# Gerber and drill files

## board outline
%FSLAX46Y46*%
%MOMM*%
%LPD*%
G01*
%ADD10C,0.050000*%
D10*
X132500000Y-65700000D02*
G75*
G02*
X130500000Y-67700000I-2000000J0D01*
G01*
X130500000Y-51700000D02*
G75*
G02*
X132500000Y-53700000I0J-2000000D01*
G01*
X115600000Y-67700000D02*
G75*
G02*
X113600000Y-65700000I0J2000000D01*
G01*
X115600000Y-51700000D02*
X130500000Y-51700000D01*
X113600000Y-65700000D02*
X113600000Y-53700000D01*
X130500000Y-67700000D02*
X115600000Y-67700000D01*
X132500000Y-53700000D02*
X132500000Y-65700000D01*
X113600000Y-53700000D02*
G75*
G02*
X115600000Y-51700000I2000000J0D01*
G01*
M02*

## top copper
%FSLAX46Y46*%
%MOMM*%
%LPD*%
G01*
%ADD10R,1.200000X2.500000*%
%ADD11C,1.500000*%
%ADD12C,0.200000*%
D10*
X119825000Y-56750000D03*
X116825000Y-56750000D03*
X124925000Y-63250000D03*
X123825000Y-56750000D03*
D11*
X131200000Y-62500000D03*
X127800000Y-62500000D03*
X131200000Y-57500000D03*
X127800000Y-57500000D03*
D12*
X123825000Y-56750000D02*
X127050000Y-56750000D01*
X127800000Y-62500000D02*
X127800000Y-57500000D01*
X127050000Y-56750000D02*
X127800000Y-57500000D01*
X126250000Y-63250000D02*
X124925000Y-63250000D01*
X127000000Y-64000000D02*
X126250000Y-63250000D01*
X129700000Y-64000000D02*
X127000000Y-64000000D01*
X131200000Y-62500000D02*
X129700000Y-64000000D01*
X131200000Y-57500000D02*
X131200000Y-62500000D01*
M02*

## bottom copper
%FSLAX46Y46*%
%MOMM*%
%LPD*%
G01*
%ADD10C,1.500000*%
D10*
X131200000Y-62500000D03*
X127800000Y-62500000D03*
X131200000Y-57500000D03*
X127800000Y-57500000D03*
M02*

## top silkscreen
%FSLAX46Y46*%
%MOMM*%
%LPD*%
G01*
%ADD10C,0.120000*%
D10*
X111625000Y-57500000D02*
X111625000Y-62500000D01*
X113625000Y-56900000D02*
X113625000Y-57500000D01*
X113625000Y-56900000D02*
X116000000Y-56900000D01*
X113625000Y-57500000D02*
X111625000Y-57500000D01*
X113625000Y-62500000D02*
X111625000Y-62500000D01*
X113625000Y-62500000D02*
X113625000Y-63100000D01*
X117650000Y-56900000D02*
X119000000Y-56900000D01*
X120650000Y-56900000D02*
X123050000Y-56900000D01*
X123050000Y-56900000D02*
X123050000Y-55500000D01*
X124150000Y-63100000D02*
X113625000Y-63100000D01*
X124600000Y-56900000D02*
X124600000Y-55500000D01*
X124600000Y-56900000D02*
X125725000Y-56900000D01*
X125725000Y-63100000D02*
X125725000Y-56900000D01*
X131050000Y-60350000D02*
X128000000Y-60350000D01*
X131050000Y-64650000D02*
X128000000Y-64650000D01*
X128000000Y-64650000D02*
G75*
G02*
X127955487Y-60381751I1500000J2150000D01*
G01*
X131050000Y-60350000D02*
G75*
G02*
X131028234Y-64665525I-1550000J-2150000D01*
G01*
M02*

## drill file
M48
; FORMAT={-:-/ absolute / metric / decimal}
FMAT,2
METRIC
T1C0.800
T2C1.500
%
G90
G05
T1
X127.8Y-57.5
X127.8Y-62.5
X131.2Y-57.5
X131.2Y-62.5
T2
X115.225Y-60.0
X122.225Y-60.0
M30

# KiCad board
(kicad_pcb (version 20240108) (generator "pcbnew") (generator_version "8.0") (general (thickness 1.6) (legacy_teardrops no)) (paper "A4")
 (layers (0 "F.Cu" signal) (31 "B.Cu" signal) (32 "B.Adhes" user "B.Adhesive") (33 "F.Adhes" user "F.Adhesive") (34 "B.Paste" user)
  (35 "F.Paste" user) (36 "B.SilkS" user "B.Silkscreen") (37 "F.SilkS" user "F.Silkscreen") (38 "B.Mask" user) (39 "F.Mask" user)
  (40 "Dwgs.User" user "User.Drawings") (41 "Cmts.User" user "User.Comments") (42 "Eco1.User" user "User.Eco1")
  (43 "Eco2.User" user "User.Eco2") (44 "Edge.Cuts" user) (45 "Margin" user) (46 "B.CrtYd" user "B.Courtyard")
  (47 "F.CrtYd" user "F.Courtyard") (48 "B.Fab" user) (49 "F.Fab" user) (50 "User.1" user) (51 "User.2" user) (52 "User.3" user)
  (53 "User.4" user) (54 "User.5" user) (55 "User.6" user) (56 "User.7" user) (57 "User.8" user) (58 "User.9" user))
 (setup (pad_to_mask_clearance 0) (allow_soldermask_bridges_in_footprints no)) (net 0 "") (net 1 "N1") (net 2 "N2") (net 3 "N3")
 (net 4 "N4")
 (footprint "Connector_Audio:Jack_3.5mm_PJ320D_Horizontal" (layer "F.Cu") (at 120 60)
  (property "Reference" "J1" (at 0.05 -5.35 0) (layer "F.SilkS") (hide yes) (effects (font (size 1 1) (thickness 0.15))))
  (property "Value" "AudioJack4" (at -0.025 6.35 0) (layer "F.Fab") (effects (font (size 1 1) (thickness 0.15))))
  (fp_line (start -8.375 -2.5) (end -8.375 2.5) (stroke (width 0.12) (type solid)) (layer "F.SilkS"))
  (fp_line (start -6.375 -3.1) (end -6.375 -2.5) (stroke (width 0.12) (type solid)) (layer "F.SilkS"))
  (fp_line (start -6.375 -3.1) (end -4 -3.1) (stroke (width 0.12) (type solid)) (layer "F.SilkS"))
  (fp_line (start -6.375 -2.5) (end -8.375 -2.5) (stroke (width 0.12) (type solid)) (layer "F.SilkS"))
  (fp_line (start -6.375 2.5) (end -8.375 2.5) (stroke (width 0.12) (type solid)) (layer "F.SilkS"))
  (fp_line (start -6.375 2.5) (end -6.375 3.1) (stroke (width 0.12) (type solid)) (layer "F.SilkS"))
  (fp_line (start -2.35 -3.1) (end -1 -3.1) (stroke (width 0.12) (type solid)) (layer "F.SilkS"))
  (fp_line (start 0.65 -3.1) (end 3.05 -3.1) (stroke (width 0.12) (type solid)) (layer "F.SilkS"))
  (fp_line (start 3.05 -3.1) (end 3.05 -4.5) (stroke (width 0.12) (type solid)) (layer "F.SilkS"))
  (fp_line (start 4.15 3.1) (end -6.375 3.1) (stroke (width 0.12) (type solid)) (layer "F.SilkS"))
  (fp_line (start 4.6 -3.1) (end 4.6 -4.5) (stroke (width 0.12) (type solid)) (layer "F.SilkS"))
  (fp_line (start 4.6 -3.1) (end 5.725 -3.1) (stroke (width 0.12) (type solid)) (layer "F.SilkS"))
  (fp_line (start 5.725 3.1) (end 5.725 -3.1) (stroke (width 0.12) (type solid)) (layer "F.SilkS"))
  (pad "" np_thru_hole circle (at -4.775 0) (size 1.5 1.5) (drill 1.5) (layers "*.Cu" "*.Mask"))
  (pad "" np_thru_hole circle (at 2.225 0) (size 1.5 1.5) (drill 1.5) (layers "*.Cu" "*.Mask"))
  (pad "R1" smd rect (at -0.175 -3.25) (size 1.2 2.5) (layers "F.Cu" "F.Paste" "F.Mask") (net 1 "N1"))
  (pad "R2" smd rect (at -3.175 -3.25) (size 1.2 2.5) (layers "F.Cu" "F.Paste" "F.Mask") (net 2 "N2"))
  (pad "S" smd rect (at 4.925 3.25) (size 1.2 2.5) (layers "F.Cu" "F.Paste" "F.Mask") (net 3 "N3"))
  (pad "T" smd rect (at 3.825 -3.25) (size 1.2 2.5) (layers "F.Cu" "F.Paste" "F.Mask") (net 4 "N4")))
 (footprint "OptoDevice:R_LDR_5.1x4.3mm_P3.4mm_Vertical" (layer "F.Cu") (at 131.2 62.5 180)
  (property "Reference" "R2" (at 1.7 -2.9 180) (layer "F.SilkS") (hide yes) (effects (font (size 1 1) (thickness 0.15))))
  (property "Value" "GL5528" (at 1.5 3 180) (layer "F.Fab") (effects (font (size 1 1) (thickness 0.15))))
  (fp_line (start 0.15 2.15) (end 3.2 2.15) (stroke (width 0.12) (type solid)) (layer "F.SilkS"))
  (fp_line (start 0.15 -2.15) (end 3.2 -2.15) (stroke (width 0.12) (type solid)) (layer "F.SilkS"))
  (fp_arc (start 3.2 -2.15) (mid 4.321403 -0.027338) (end 3.244513 2.118249) (stroke (width 0.12) (type solid)) (layer "F.SilkS"))
  (fp_arc (start 0.15 2.15) (mid -0.950438 -0.013368) (end 0.171766 -2.165525) (stroke (width 0.12) (type solid)) (layer "F.SilkS"))
  (pad "1" thru_hole circle (at 0 0 180) (size 1.5 1.5) (drill 0.8) (layers "*.Cu" "*.Mask") (remove_unused_layers no) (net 3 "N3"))
  (pad "2" thru_hole circle (at 3.4 0 180) (size 1.5 1.5) (drill 0.8) (layers "*.Cu" "*.Mask") (remove_unused_layers no) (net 4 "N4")))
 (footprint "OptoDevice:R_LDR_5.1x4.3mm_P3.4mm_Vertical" (layer "B.Cu") (at 131.2 57.5 180)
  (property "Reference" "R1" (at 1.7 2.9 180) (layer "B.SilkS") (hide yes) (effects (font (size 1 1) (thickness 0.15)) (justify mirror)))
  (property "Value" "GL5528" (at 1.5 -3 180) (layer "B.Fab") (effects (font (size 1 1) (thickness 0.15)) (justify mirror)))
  (pad "1" thru_hole circle (at 0 0 180) (size 1.5 1.5) (drill 0.8) (layers "*.Cu" "*.Mask") (remove_unused_layers no) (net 3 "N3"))
  (pad "2" thru_hole circle (at 3.4 0 180) (size 1.5 1.5) (drill 0.8) (layers "*.Cu" "*.Mask") (remove_unused_layers no) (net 4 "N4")))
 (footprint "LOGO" (layer "B.Cu") (at 120.6 55.7 180)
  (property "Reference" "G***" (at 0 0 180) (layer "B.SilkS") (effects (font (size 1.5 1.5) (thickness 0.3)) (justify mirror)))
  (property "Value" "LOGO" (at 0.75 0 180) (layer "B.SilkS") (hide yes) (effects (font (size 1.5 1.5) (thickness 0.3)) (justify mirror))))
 (gr_arc (start 132.5 65.7) (mid 131.914214 67.114214) (end 130.5 67.7) (stroke (width 0.05) (type default)) (layer "Edge.Cuts"))
 (gr_arc (start 130.5 51.7) (mid 131.914214 52.285786) (end 132.5 53.7) (stroke (width 0.05) (type default)) (layer "Edge.Cuts"))
 (gr_arc (start 115.6 67.7) (mid 114.185786 67.114214) (end 113.6 65.7) (stroke (width 0.05) (type default)) (layer "Edge.Cuts"))
 (gr_line (start 115.6 51.7) (end 130.5 51.7) (stroke (width 0.05) (type default)) (layer "Edge.Cuts"))
 (gr_line (start 113.6 65.7) (end 113.6 53.7) (stroke (width 0.05) (type default)) (layer "Edge.Cuts"))
 (gr_line (start 130.5 67.7) (end 115.6 67.7) (stroke (width 0.05) (type default)) (layer "Edge.Cuts"))
 (gr_line (start 132.5 53.7) (end 132.5 65.7) (stroke (width 0.05) (type default)) (layer "Edge.Cuts"))
 (gr_arc (start 113.6 53.7) (mid 114.185786 52.285786) (end 115.6 51.7) (stroke (width 0.05) (type default)) (layer "Edge.Cuts"))
 (segment (start 123.825 56.75) (end 127.05 56.75) (width 0.2) (layer "F.Cu") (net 4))
 (segment (start 127.8 62.5) (end 127.8 57.5) (width 0.2) (layer "F.Cu") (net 4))
 (segment (start 127.05 56.75) (end 127.8 57.5) (width 0.2) (layer "F.Cu") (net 4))
 (segment (start 126.25 63.25) (end 124.925 63.25) (width 0.2) (layer "F.Cu") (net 3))
 (segment (start 127 64) (end 126.25 63.25) (width 0.2) (layer "F.Cu") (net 3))
 (segment (start 129.7 64) (end 127 64) (width 0.2) (layer "F.Cu") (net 3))
 (segment (start 131.2 62.5) (end 129.7 64) (width 0.2) (layer "F.Cu") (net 3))
 (segment (start 131.2 57.5) (end 131.2 62.5) (width 0.2) (layer "F.Cu") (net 3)))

